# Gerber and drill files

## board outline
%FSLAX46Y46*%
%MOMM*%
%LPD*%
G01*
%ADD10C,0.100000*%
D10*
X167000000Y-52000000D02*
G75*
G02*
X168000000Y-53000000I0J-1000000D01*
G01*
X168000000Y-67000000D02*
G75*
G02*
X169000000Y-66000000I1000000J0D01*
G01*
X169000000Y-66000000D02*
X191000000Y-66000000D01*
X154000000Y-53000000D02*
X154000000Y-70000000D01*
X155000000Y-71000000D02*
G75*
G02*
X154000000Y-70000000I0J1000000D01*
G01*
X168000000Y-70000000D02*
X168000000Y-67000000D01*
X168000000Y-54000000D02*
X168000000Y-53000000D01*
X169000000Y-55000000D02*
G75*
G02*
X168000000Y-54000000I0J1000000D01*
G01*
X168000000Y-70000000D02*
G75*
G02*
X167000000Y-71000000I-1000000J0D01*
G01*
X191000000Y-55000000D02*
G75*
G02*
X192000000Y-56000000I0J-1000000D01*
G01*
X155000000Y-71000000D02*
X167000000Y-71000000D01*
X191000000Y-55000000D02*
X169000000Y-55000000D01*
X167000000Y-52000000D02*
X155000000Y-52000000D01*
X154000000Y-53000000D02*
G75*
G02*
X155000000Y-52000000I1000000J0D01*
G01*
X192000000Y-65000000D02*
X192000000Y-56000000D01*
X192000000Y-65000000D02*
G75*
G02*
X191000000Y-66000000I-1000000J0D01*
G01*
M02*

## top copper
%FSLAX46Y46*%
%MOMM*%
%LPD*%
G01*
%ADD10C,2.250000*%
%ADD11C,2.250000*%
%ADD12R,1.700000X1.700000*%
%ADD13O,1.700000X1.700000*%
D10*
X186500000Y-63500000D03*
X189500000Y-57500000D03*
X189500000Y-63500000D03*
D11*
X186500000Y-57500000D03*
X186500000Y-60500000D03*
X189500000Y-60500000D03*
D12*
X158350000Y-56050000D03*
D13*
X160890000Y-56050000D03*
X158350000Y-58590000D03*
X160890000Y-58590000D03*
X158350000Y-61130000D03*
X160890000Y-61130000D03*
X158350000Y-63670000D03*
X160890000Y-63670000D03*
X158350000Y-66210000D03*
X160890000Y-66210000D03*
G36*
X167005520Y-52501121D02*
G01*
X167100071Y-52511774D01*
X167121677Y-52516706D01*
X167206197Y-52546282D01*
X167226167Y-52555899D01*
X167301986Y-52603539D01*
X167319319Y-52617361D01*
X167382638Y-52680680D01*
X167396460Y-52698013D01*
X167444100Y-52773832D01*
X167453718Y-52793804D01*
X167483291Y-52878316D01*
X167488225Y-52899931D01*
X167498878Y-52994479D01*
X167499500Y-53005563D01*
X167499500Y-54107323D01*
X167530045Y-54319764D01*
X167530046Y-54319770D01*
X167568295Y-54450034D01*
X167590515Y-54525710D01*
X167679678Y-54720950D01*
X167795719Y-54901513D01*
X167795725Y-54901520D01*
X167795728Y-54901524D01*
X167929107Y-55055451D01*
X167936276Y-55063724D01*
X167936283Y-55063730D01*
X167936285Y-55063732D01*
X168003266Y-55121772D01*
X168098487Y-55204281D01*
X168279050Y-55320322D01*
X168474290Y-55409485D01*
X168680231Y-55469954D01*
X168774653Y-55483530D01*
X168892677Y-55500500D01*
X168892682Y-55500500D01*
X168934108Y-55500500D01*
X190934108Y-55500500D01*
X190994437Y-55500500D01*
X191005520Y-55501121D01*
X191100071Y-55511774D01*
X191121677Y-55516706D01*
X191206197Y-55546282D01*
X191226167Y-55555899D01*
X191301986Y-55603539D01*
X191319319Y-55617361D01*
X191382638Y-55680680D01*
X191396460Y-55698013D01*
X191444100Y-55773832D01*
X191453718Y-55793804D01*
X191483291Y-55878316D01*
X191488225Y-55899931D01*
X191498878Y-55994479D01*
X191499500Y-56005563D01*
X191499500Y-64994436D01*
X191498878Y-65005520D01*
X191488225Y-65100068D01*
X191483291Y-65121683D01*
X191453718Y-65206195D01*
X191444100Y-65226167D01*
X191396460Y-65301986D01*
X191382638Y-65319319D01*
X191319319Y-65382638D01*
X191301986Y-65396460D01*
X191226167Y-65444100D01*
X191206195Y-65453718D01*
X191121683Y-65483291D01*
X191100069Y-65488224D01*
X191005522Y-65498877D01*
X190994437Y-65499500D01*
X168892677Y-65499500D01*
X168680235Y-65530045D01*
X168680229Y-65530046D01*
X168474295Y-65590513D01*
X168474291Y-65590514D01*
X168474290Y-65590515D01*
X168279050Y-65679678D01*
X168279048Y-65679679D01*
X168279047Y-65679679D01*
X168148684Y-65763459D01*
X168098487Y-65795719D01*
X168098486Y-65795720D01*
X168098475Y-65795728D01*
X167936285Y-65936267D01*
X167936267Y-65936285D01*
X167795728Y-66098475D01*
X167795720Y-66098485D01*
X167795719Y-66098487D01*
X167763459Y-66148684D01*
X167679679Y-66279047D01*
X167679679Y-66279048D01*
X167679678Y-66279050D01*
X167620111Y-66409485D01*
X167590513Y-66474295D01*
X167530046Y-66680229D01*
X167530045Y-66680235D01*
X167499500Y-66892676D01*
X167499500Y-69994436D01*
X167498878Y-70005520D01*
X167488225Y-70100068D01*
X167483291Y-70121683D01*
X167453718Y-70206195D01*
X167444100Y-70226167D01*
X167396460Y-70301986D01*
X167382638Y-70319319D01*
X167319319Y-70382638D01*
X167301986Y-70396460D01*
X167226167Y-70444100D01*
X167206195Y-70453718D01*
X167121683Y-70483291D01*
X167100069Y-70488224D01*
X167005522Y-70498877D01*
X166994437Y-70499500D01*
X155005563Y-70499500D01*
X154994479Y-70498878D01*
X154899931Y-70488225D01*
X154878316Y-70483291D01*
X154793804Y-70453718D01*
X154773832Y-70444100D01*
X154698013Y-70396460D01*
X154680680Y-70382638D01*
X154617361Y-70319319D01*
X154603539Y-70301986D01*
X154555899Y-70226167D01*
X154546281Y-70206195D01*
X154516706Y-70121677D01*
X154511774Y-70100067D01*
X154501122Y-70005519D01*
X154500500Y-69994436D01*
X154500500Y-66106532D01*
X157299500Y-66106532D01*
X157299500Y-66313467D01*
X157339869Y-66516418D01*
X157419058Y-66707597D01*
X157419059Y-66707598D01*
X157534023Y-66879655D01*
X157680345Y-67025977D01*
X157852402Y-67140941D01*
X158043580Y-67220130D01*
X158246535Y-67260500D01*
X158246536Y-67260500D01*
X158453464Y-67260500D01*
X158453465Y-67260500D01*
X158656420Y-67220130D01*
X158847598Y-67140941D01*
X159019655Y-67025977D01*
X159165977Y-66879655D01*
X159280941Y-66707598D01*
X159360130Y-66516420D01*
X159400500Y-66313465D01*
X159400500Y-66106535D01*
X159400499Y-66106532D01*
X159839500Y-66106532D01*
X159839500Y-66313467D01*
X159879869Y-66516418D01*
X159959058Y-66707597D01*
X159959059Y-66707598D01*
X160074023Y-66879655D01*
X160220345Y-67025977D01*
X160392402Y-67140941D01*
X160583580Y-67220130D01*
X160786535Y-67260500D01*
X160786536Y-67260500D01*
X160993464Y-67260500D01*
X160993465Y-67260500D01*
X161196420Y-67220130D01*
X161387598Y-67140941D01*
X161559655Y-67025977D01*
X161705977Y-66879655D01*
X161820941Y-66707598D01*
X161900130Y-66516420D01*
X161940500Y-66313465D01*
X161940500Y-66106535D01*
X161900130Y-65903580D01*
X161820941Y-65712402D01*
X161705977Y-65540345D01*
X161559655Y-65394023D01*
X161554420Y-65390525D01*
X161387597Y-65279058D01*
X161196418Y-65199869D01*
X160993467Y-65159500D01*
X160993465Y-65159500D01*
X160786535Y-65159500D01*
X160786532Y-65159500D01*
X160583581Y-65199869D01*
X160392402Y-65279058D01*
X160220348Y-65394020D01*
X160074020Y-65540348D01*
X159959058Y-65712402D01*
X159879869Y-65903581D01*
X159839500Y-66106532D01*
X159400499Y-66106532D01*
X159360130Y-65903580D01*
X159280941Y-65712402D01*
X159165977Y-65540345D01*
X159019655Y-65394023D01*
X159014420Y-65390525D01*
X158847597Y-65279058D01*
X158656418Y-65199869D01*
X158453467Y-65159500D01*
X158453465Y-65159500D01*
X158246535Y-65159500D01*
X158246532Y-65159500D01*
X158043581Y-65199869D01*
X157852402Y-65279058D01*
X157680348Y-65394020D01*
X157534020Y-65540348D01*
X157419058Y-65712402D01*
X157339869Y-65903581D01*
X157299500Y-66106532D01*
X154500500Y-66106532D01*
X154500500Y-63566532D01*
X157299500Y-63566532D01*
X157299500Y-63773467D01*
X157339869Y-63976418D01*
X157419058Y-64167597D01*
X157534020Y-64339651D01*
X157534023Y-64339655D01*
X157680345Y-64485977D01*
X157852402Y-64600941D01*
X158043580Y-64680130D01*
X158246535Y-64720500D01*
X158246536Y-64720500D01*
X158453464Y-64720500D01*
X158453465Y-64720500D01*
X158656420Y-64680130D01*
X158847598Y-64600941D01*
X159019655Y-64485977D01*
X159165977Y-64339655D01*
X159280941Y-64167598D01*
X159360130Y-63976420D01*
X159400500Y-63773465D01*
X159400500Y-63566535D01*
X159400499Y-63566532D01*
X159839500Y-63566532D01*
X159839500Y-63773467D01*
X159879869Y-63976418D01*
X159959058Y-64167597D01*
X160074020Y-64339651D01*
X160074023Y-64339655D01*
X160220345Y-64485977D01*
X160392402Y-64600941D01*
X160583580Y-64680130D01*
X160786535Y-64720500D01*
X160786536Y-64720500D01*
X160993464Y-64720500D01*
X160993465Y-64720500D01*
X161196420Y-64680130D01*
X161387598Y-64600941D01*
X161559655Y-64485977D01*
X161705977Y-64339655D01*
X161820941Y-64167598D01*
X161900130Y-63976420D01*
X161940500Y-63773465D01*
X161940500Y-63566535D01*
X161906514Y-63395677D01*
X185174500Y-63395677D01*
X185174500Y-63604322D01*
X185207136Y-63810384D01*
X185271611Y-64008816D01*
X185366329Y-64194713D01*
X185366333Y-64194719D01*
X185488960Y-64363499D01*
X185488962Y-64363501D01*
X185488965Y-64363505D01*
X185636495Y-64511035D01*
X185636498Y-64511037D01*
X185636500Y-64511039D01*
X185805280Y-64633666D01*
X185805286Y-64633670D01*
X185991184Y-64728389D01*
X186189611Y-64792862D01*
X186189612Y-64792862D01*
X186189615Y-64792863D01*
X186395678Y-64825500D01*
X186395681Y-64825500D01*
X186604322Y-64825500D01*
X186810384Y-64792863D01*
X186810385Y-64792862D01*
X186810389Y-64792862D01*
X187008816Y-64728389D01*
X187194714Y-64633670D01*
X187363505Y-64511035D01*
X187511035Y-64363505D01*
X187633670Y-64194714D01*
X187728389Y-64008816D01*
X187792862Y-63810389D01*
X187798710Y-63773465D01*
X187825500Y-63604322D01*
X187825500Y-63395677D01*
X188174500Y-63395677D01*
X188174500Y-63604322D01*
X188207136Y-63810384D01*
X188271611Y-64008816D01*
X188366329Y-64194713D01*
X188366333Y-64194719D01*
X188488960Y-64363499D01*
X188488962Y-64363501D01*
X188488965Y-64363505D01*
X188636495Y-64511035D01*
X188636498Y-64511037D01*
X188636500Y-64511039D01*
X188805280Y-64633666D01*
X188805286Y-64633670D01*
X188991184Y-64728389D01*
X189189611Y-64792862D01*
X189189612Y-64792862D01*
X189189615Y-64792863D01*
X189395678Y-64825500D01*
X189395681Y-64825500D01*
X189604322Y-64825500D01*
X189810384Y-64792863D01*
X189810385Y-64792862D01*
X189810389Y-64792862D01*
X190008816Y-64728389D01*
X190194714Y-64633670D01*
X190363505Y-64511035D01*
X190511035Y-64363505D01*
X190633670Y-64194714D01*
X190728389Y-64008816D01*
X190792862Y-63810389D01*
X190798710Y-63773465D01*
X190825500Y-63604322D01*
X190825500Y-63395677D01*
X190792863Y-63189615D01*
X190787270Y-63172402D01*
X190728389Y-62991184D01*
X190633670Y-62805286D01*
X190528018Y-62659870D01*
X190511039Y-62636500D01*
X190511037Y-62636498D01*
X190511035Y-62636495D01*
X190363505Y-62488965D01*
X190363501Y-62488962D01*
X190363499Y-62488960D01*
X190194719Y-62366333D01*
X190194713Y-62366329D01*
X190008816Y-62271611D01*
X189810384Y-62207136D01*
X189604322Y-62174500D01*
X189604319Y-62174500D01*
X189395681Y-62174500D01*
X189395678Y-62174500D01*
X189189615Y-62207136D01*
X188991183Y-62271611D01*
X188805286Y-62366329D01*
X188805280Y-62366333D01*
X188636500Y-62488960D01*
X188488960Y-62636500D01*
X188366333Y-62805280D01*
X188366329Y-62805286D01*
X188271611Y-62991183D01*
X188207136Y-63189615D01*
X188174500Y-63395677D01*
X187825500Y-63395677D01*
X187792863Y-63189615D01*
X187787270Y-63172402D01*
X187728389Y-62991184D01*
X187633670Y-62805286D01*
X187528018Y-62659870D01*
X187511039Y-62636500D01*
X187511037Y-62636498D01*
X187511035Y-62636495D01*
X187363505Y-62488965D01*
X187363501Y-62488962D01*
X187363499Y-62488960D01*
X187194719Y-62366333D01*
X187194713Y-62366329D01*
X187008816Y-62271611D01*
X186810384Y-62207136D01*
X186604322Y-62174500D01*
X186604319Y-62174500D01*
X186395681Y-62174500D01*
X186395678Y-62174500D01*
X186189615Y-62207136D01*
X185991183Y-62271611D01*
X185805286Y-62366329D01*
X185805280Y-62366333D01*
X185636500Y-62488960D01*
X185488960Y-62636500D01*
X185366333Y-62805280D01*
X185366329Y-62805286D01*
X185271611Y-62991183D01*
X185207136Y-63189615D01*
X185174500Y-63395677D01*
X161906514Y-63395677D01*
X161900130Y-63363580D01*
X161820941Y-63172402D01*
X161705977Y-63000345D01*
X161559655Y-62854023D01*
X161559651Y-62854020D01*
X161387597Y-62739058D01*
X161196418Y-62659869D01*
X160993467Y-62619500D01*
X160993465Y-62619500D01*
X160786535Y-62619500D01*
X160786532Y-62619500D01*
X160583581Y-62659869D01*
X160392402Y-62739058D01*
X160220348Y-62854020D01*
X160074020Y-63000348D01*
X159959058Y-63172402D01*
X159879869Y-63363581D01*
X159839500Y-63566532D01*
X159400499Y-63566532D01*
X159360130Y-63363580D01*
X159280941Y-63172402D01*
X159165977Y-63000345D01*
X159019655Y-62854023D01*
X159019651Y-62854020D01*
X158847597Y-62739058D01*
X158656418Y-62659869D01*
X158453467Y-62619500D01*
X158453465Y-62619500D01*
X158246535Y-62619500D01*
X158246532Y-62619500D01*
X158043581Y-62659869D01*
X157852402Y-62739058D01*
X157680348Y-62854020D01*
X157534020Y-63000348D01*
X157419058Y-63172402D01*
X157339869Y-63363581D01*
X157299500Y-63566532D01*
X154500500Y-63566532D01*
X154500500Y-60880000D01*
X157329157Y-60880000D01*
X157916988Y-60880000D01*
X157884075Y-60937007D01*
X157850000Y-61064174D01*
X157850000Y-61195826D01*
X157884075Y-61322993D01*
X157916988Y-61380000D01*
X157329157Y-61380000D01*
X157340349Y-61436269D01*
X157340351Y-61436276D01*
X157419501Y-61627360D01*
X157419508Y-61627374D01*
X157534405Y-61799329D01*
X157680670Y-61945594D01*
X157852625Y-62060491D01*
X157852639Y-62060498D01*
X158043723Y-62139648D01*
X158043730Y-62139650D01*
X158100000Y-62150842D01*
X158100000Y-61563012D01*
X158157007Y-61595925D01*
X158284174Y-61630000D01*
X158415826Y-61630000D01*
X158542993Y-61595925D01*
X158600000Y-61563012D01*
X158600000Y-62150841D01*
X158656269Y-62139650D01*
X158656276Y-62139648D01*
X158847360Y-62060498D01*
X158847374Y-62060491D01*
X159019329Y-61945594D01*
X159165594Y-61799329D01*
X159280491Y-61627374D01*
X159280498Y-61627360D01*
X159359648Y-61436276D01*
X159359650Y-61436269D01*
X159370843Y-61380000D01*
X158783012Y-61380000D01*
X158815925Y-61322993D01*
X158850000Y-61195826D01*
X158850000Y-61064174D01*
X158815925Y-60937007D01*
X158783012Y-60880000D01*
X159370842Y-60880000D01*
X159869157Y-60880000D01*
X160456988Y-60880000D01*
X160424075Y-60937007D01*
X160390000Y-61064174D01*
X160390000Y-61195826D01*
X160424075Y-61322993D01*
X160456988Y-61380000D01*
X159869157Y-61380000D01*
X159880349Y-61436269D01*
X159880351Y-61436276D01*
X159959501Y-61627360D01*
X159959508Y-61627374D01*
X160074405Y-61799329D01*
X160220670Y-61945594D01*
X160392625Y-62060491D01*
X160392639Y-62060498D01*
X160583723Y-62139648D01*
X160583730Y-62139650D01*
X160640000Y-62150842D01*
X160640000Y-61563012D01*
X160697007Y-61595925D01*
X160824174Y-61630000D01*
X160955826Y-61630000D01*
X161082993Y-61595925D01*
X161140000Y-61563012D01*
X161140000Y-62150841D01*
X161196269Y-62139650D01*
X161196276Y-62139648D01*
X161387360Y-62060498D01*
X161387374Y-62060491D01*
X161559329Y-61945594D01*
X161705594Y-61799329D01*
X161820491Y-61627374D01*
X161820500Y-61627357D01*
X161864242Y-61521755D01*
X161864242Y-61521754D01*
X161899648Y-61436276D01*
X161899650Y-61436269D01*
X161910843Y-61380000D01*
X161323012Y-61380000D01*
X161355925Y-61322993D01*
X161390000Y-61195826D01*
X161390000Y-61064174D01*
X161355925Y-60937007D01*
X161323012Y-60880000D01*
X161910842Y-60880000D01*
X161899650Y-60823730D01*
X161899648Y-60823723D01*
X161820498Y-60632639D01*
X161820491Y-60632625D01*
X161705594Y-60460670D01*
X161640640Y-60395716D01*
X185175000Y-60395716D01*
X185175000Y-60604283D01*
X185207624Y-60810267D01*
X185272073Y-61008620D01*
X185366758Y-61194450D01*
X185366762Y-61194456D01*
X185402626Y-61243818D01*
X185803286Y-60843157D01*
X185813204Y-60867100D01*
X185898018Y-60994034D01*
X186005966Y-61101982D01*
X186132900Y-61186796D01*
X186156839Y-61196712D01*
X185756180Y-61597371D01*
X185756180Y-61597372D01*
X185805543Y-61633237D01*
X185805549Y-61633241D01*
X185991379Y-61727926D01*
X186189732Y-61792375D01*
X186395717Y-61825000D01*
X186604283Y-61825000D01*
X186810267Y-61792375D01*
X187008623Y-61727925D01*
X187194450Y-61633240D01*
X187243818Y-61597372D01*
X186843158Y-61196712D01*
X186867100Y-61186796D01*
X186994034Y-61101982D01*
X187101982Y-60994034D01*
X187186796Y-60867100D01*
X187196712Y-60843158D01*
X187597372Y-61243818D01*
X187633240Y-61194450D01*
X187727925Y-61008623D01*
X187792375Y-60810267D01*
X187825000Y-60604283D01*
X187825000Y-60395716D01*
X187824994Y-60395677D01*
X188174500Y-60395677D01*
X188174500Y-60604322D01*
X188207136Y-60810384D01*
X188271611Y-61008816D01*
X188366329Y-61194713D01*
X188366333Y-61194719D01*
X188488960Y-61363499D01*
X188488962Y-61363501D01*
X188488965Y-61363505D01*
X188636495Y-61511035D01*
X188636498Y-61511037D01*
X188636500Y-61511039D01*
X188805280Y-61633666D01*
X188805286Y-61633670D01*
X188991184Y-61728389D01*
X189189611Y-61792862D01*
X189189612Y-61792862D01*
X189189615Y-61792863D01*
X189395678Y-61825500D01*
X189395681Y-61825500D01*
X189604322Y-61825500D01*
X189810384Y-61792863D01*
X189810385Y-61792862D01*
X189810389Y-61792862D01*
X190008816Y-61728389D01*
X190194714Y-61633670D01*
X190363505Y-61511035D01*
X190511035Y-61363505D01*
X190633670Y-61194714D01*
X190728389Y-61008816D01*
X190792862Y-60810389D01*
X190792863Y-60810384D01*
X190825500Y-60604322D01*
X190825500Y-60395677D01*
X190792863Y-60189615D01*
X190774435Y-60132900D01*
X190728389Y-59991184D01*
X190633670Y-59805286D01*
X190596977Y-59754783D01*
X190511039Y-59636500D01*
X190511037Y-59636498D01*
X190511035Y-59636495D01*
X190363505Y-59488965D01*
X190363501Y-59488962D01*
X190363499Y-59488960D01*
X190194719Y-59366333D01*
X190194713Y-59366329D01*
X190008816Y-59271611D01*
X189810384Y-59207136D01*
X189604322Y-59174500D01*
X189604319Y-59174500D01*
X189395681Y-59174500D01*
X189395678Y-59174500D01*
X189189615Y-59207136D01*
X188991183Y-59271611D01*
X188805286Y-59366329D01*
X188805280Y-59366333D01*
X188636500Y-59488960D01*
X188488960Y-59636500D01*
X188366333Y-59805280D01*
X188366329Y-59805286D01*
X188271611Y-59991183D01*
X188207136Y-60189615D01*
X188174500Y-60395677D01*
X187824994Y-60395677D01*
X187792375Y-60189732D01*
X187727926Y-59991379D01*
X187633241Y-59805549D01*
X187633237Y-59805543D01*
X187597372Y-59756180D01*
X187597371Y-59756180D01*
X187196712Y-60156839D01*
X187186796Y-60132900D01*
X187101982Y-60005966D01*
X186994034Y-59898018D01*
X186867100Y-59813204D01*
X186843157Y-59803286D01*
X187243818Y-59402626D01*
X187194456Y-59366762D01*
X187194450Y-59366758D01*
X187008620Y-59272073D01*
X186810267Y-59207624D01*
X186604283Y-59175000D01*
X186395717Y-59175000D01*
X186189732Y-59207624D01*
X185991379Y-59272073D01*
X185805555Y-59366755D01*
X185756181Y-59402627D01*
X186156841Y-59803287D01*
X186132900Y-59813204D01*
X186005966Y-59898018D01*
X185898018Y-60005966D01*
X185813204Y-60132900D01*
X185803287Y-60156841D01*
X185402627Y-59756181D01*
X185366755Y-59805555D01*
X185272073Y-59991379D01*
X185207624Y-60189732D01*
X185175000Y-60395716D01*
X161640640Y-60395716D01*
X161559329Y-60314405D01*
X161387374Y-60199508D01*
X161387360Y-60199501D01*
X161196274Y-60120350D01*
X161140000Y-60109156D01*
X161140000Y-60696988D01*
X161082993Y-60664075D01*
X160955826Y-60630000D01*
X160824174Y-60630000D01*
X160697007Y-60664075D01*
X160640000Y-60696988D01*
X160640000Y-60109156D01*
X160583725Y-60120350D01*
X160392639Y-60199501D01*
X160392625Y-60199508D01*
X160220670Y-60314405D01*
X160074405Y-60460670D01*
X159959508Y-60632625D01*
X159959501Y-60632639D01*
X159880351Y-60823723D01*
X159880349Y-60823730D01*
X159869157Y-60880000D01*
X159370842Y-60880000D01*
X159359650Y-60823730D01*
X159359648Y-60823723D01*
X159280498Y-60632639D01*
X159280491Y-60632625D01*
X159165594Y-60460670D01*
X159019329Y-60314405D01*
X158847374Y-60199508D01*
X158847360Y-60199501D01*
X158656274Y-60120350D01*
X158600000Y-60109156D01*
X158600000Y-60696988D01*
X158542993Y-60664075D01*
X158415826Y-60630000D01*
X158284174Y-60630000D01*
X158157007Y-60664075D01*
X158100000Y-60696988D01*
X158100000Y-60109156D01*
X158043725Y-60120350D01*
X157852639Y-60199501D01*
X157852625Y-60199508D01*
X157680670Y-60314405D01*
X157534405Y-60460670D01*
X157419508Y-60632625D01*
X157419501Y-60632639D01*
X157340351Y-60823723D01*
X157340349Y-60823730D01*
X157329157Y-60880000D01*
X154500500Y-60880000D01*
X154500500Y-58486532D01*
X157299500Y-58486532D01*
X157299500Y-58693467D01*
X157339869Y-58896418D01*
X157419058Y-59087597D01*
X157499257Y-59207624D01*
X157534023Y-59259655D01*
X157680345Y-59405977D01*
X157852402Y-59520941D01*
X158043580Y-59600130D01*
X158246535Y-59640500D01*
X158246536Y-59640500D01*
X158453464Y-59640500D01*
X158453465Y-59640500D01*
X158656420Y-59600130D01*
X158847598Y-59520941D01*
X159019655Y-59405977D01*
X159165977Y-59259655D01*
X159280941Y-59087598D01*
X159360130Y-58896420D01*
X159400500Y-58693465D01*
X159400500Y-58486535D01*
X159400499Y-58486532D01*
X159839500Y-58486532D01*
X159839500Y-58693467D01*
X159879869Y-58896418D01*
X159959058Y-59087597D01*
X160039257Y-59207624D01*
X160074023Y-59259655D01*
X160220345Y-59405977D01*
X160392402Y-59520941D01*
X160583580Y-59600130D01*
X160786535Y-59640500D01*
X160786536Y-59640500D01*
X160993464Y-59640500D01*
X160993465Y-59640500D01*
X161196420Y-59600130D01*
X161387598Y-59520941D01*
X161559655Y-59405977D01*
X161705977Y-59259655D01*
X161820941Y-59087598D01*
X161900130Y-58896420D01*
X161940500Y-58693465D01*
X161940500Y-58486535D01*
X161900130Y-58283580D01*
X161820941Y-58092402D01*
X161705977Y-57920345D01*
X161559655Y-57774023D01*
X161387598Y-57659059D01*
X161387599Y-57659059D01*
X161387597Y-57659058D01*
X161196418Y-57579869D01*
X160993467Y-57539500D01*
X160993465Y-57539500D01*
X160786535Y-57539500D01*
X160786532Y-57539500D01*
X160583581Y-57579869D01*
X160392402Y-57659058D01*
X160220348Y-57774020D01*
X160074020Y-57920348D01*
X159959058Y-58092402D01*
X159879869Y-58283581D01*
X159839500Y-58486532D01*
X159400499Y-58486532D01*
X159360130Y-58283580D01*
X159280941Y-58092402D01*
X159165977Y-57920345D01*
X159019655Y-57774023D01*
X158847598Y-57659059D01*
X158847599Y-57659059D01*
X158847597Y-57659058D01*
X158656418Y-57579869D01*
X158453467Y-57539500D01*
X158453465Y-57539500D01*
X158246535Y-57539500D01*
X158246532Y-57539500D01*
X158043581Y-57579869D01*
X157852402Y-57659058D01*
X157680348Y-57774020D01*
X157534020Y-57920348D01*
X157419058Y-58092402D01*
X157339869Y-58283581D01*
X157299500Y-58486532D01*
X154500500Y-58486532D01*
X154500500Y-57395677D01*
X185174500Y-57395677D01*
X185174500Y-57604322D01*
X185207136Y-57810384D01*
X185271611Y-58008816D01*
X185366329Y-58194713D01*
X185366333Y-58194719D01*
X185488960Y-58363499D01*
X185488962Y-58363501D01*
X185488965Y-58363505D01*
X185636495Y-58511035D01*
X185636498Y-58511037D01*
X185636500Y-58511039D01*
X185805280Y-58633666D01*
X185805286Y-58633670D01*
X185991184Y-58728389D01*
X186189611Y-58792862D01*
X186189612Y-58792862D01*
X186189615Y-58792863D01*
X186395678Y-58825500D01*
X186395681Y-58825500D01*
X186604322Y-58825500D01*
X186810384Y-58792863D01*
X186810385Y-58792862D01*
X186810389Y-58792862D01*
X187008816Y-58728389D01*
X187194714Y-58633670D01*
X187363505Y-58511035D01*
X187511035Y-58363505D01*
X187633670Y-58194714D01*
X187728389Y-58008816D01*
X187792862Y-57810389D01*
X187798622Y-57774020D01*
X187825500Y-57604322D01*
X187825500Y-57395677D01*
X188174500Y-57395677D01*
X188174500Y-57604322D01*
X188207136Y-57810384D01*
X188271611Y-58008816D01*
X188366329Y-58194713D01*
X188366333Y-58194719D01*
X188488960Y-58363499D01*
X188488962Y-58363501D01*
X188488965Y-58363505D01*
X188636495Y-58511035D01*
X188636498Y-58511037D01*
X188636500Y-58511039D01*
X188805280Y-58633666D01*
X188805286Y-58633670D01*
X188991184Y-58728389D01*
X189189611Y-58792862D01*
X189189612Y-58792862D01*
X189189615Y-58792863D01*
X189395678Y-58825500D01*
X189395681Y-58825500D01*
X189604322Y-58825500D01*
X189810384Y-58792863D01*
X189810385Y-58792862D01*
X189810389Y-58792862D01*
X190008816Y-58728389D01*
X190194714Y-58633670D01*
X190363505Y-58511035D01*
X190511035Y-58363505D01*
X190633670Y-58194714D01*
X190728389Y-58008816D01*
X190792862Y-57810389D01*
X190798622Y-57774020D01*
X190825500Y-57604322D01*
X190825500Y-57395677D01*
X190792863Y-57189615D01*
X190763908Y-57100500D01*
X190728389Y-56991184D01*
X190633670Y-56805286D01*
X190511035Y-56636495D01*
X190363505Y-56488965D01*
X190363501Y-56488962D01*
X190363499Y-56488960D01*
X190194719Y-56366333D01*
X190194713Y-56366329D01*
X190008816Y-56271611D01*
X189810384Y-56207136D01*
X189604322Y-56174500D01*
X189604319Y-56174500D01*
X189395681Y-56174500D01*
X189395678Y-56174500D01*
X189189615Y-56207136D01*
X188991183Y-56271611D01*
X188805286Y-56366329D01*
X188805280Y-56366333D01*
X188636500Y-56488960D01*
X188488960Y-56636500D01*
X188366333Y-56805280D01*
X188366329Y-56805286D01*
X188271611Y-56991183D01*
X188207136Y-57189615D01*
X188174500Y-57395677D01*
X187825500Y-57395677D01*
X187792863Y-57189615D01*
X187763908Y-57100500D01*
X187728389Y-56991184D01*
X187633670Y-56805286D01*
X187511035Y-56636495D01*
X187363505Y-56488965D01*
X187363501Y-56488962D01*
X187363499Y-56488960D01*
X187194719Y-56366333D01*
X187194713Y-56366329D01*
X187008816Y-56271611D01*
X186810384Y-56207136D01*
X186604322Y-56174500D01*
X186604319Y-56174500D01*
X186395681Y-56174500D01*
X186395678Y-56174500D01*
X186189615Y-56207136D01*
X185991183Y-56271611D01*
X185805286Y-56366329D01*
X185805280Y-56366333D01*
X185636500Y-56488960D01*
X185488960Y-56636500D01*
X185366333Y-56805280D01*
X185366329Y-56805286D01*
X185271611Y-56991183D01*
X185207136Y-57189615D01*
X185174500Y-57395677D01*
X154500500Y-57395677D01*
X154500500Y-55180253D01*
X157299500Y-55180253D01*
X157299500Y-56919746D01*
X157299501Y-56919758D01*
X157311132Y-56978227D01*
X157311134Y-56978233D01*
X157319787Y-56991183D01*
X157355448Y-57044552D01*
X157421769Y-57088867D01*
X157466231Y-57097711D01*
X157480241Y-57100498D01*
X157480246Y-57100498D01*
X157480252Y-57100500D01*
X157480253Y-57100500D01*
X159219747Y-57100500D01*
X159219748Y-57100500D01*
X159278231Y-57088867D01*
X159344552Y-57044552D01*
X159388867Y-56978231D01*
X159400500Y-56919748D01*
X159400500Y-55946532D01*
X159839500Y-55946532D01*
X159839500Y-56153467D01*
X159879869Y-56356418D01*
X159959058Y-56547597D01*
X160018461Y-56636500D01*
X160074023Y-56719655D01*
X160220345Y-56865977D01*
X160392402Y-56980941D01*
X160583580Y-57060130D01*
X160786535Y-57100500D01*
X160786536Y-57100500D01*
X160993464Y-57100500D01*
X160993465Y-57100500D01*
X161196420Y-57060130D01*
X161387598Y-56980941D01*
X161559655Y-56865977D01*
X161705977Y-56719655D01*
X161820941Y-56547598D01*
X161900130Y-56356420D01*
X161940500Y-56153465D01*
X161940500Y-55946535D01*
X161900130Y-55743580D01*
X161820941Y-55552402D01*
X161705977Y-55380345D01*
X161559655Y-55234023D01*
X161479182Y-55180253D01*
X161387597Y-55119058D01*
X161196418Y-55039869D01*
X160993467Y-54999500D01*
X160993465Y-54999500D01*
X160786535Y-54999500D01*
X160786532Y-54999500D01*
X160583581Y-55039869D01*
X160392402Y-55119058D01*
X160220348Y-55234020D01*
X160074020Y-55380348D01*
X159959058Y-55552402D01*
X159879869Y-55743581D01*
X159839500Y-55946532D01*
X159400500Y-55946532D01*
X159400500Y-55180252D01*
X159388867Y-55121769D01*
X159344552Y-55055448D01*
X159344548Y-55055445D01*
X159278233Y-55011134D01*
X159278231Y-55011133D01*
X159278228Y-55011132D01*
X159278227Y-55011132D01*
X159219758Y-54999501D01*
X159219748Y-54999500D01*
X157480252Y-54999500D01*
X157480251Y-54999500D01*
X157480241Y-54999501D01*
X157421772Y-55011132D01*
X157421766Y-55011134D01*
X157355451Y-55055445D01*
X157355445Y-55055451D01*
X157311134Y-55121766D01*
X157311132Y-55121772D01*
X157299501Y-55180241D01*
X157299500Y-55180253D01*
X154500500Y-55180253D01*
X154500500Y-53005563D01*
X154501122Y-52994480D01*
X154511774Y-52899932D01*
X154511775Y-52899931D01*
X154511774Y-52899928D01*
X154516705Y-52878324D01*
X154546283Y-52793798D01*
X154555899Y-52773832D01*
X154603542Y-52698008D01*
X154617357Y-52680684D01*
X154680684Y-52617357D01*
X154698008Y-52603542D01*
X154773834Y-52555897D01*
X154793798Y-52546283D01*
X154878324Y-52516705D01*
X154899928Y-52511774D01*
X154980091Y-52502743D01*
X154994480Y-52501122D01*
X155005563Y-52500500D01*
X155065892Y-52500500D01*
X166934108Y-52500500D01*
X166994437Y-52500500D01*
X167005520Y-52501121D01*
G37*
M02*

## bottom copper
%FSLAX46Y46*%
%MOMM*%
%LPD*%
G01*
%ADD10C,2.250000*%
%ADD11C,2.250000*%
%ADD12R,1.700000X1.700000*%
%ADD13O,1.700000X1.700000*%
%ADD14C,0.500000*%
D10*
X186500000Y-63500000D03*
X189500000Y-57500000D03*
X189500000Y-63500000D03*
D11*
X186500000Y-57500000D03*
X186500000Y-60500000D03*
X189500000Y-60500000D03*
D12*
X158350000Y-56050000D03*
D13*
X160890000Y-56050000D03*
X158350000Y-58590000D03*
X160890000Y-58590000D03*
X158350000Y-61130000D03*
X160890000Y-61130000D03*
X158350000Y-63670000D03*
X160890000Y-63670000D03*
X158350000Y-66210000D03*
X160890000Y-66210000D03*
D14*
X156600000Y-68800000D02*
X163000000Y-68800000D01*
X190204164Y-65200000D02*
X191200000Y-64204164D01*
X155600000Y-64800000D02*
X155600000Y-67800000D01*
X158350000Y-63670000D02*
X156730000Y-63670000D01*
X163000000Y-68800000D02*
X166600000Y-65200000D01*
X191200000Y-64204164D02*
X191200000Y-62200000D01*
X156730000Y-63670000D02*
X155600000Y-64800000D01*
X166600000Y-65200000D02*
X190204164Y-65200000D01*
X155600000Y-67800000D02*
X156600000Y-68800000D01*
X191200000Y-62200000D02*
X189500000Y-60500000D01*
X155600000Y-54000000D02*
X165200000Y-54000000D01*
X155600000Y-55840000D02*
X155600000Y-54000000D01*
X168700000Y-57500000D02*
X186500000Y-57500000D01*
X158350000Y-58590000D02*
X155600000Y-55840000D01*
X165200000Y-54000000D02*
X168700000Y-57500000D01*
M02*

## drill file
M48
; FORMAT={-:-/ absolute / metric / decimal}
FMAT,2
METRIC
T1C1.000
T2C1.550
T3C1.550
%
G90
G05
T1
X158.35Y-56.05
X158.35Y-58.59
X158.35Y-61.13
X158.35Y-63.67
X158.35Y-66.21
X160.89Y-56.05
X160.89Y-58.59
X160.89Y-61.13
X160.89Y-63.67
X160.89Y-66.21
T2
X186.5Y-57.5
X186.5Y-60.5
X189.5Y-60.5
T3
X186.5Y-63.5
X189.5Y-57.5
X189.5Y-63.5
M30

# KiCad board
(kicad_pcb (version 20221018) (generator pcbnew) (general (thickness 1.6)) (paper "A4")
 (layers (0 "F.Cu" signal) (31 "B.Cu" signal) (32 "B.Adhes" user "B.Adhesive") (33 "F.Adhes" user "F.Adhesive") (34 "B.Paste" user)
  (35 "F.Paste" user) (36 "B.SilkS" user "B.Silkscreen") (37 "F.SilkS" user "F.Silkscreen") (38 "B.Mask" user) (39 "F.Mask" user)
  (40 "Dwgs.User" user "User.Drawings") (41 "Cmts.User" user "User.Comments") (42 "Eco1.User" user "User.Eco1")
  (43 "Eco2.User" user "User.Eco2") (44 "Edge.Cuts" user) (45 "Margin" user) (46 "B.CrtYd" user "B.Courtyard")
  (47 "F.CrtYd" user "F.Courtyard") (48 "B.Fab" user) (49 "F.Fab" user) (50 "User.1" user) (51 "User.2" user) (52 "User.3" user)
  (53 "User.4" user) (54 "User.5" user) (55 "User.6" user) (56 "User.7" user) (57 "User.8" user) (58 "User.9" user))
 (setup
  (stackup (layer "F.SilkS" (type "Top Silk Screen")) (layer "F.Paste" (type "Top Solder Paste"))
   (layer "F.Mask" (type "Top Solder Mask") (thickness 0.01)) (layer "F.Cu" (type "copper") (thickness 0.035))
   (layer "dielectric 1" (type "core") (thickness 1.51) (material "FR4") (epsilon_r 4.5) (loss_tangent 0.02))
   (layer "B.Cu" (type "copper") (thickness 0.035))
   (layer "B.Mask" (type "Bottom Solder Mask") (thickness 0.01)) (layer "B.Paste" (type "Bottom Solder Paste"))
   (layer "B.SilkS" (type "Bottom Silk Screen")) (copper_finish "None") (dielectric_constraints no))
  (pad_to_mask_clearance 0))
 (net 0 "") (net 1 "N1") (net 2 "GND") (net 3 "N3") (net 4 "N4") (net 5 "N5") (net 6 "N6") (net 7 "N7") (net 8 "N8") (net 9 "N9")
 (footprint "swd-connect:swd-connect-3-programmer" (layer "F.Cu") (at 188 60.5)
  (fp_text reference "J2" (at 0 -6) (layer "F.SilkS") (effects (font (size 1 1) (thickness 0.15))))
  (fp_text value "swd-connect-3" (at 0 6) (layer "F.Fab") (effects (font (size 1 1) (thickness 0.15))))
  (pad "" np_thru_hole circle (at -1.5 3) (size 2.25 2.25) (drill 1.55) (layers "F&B.Cu" "*.Mask"))
  (pad "" np_thru_hole circle (at 1.5 -3) (size 2.25 2.25) (drill 1.55) (layers "F&B.Cu" "*.Mask"))
  (pad "" np_thru_hole circle (at 1.5 3) (size 2.25 2.25) (drill 1.55) (layers "F&B.Cu" "*.Mask"))
  (pad "1" thru_hole circle (at -1.5 -3) (size 2.25 2.25) (drill 1.55) (layers "*.Cu" "*.Mask") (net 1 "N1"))
  (pad "2" thru_hole circle (at -1.5 0) (size 2.25 2.25) (drill 1.55) (layers "*.Cu" "*.Mask") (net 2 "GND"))
  (pad "3" thru_hole circle (at 1.5 0) (size 2.25 2.25) (drill 1.55) (layers "*.Cu" "*.Mask") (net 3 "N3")))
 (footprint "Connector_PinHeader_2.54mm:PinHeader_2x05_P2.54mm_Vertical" (layer "F.Cu") (at 158.35 56.05)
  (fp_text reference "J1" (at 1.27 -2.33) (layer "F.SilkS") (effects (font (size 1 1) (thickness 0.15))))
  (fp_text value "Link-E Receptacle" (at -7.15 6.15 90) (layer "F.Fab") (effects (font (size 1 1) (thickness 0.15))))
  (pad "1" thru_hole rect (at 0 0) (size 1.7 1.7) (drill 1) (layers "*.Cu" "*.Mask") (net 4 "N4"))
  (pad "2" thru_hole oval (at 2.54 0) (size 1.7 1.7) (drill 1) (layers "*.Cu" "*.Mask") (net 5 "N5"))
  (pad "3" thru_hole oval (at 0 2.54) (size 1.7 1.7) (drill 1) (layers "*.Cu" "*.Mask") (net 1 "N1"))
  (pad "4" thru_hole oval (at 2.54 2.54) (size 1.7 1.7) (drill 1) (layers "*.Cu" "*.Mask") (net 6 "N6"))
  (pad "5" thru_hole oval (at 0 5.08) (size 1.7 1.7) (drill 1) (layers "*.Cu" "*.Mask") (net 2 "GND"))
  (pad "6" thru_hole oval (at 2.54 5.08) (size 1.7 1.7) (drill 1) (layers "*.Cu" "*.Mask") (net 2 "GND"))
  (pad "7" thru_hole oval (at 0 7.62) (size 1.7 1.7) (drill 1) (layers "*.Cu" "*.Mask") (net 3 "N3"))
  (pad "8" thru_hole oval (at 2.54 7.62) (size 1.7 1.7) (drill 1) (layers "*.Cu" "*.Mask") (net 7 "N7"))
  (pad "9" thru_hole oval (at 0 10.16) (size 1.7 1.7) (drill 1) (layers "*.Cu" "*.Mask") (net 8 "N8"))
  (pad "10" thru_hole oval (at 2.54 10.16) (size 1.7 1.7) (drill 1) (layers "*.Cu" "*.Mask") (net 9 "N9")))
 (gr_arc (start 167 52) (mid 167.707107 52.292893) (end 168 53) (stroke (width 0.1) (type default)) (layer "Edge.Cuts"))
 (gr_arc (start 168 67) (mid 168.292893 66.292893) (end 169 66) (stroke (width 0.1) (type default)) (layer "Edge.Cuts"))
 (gr_line (start 169 66) (end 191 66) (stroke (width 0.1) (type default)) (layer "Edge.Cuts"))
 (gr_line (start 154 53) (end 154 70) (stroke (width 0.1) (type default)) (layer "Edge.Cuts"))
 (gr_arc (start 155 71) (mid 154.292893 70.707107) (end 154 70) (stroke (width 0.1) (type default)) (layer "Edge.Cuts"))
 (gr_line (start 168 70) (end 168 67) (stroke (width 0.1) (type default)) (layer "Edge.Cuts"))
 (gr_line (start 168 54) (end 168 53) (stroke (width 0.1) (type default)) (layer "Edge.Cuts"))
 (gr_arc (start 169 55) (mid 168.292893 54.707107) (end 168 54) (stroke (width 0.1) (type default)) (layer "Edge.Cuts"))
 (gr_arc (start 168 70) (mid 167.707107 70.707107) (end 167 71) (stroke (width 0.1) (type default)) (layer "Edge.Cuts"))
 (gr_arc (start 191 55) (mid 191.707107 55.292893) (end 192 56) (stroke (width 0.1) (type default)) (layer "Edge.Cuts"))
 (gr_line (start 155 71) (end 167 71) (stroke (width 0.1) (type default)) (layer "Edge.Cuts"))
 (gr_line (start 191 55) (end 169 55) (stroke (width 0.1) (type default)) (layer "Edge.Cuts"))
 (gr_line (start 167 52) (end 155 52) (stroke (width 0.1) (type default)) (layer "Edge.Cuts"))
 (gr_arc (start 154 53) (mid 154.292893 52.292893) (end 155 52) (stroke (width 0.1) (type default)) (layer "Edge.Cuts"))
 (gr_line (start 192 65) (end 192 56) (stroke (width 0.1) (type default)) (layer "Edge.Cuts"))
 (gr_arc (start 192 65) (mid 191.707107 65.707107) (end 191 66) (stroke (width 0.1) (type default)) (layer "Edge.Cuts"))
 (segment (start 156.6 68.8) (end 163 68.8) (width 0.5) (layer "B.Cu") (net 3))
 (segment (start 190.204164 65.2) (end 191.2 64.204164) (width 0.5) (layer "B.Cu") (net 3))
 (segment (start 155.6 64.8) (end 155.6 67.8) (width 0.5) (layer "B.Cu") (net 3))
 (segment (start 158.35 63.67) (end 156.73 63.67) (width 0.5) (layer "B.Cu") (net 3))
 (segment (start 163 68.8) (end 166.6 65.2) (width 0.5) (layer "B.Cu") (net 3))
 (segment (start 191.2 64.204164) (end 191.2 62.2) (width 0.5) (layer "B.Cu") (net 3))
 (segment (start 156.73 63.67) (end 155.6 64.8) (width 0.5) (layer "B.Cu") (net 3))
 (segment (start 166.6 65.2) (end 190.204164 65.2) (width 0.5) (layer "B.Cu") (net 3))
 (segment (start 155.6 67.8) (end 156.6 68.8) (width 0.5) (layer "B.Cu") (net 3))
 (segment (start 191.2 62.2) (end 189.5 60.5) (width 0.5) (layer "B.Cu") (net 3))
 (segment (start 155.6 54) (end 165.2 54) (width 0.5) (layer "B.Cu") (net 1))
 (segment (start 155.6 55.84) (end 155.6 54) (width 0.5) (layer "B.Cu") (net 1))
 (segment (start 168.7 57.5) (end 186.5 57.5) (width 0.5) (layer "B.Cu") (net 1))
 (segment (start 158.35 58.59) (end 155.6 55.84) (width 0.5) (layer "B.Cu") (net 1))
 (segment (start 165.2 54) (end 168.7 57.5) (width 0.5) (layer "B.Cu") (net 1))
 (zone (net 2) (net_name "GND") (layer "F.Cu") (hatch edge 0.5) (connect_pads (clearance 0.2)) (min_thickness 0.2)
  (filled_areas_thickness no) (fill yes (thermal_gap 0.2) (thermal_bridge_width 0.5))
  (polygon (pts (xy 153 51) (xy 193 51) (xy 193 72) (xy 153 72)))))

